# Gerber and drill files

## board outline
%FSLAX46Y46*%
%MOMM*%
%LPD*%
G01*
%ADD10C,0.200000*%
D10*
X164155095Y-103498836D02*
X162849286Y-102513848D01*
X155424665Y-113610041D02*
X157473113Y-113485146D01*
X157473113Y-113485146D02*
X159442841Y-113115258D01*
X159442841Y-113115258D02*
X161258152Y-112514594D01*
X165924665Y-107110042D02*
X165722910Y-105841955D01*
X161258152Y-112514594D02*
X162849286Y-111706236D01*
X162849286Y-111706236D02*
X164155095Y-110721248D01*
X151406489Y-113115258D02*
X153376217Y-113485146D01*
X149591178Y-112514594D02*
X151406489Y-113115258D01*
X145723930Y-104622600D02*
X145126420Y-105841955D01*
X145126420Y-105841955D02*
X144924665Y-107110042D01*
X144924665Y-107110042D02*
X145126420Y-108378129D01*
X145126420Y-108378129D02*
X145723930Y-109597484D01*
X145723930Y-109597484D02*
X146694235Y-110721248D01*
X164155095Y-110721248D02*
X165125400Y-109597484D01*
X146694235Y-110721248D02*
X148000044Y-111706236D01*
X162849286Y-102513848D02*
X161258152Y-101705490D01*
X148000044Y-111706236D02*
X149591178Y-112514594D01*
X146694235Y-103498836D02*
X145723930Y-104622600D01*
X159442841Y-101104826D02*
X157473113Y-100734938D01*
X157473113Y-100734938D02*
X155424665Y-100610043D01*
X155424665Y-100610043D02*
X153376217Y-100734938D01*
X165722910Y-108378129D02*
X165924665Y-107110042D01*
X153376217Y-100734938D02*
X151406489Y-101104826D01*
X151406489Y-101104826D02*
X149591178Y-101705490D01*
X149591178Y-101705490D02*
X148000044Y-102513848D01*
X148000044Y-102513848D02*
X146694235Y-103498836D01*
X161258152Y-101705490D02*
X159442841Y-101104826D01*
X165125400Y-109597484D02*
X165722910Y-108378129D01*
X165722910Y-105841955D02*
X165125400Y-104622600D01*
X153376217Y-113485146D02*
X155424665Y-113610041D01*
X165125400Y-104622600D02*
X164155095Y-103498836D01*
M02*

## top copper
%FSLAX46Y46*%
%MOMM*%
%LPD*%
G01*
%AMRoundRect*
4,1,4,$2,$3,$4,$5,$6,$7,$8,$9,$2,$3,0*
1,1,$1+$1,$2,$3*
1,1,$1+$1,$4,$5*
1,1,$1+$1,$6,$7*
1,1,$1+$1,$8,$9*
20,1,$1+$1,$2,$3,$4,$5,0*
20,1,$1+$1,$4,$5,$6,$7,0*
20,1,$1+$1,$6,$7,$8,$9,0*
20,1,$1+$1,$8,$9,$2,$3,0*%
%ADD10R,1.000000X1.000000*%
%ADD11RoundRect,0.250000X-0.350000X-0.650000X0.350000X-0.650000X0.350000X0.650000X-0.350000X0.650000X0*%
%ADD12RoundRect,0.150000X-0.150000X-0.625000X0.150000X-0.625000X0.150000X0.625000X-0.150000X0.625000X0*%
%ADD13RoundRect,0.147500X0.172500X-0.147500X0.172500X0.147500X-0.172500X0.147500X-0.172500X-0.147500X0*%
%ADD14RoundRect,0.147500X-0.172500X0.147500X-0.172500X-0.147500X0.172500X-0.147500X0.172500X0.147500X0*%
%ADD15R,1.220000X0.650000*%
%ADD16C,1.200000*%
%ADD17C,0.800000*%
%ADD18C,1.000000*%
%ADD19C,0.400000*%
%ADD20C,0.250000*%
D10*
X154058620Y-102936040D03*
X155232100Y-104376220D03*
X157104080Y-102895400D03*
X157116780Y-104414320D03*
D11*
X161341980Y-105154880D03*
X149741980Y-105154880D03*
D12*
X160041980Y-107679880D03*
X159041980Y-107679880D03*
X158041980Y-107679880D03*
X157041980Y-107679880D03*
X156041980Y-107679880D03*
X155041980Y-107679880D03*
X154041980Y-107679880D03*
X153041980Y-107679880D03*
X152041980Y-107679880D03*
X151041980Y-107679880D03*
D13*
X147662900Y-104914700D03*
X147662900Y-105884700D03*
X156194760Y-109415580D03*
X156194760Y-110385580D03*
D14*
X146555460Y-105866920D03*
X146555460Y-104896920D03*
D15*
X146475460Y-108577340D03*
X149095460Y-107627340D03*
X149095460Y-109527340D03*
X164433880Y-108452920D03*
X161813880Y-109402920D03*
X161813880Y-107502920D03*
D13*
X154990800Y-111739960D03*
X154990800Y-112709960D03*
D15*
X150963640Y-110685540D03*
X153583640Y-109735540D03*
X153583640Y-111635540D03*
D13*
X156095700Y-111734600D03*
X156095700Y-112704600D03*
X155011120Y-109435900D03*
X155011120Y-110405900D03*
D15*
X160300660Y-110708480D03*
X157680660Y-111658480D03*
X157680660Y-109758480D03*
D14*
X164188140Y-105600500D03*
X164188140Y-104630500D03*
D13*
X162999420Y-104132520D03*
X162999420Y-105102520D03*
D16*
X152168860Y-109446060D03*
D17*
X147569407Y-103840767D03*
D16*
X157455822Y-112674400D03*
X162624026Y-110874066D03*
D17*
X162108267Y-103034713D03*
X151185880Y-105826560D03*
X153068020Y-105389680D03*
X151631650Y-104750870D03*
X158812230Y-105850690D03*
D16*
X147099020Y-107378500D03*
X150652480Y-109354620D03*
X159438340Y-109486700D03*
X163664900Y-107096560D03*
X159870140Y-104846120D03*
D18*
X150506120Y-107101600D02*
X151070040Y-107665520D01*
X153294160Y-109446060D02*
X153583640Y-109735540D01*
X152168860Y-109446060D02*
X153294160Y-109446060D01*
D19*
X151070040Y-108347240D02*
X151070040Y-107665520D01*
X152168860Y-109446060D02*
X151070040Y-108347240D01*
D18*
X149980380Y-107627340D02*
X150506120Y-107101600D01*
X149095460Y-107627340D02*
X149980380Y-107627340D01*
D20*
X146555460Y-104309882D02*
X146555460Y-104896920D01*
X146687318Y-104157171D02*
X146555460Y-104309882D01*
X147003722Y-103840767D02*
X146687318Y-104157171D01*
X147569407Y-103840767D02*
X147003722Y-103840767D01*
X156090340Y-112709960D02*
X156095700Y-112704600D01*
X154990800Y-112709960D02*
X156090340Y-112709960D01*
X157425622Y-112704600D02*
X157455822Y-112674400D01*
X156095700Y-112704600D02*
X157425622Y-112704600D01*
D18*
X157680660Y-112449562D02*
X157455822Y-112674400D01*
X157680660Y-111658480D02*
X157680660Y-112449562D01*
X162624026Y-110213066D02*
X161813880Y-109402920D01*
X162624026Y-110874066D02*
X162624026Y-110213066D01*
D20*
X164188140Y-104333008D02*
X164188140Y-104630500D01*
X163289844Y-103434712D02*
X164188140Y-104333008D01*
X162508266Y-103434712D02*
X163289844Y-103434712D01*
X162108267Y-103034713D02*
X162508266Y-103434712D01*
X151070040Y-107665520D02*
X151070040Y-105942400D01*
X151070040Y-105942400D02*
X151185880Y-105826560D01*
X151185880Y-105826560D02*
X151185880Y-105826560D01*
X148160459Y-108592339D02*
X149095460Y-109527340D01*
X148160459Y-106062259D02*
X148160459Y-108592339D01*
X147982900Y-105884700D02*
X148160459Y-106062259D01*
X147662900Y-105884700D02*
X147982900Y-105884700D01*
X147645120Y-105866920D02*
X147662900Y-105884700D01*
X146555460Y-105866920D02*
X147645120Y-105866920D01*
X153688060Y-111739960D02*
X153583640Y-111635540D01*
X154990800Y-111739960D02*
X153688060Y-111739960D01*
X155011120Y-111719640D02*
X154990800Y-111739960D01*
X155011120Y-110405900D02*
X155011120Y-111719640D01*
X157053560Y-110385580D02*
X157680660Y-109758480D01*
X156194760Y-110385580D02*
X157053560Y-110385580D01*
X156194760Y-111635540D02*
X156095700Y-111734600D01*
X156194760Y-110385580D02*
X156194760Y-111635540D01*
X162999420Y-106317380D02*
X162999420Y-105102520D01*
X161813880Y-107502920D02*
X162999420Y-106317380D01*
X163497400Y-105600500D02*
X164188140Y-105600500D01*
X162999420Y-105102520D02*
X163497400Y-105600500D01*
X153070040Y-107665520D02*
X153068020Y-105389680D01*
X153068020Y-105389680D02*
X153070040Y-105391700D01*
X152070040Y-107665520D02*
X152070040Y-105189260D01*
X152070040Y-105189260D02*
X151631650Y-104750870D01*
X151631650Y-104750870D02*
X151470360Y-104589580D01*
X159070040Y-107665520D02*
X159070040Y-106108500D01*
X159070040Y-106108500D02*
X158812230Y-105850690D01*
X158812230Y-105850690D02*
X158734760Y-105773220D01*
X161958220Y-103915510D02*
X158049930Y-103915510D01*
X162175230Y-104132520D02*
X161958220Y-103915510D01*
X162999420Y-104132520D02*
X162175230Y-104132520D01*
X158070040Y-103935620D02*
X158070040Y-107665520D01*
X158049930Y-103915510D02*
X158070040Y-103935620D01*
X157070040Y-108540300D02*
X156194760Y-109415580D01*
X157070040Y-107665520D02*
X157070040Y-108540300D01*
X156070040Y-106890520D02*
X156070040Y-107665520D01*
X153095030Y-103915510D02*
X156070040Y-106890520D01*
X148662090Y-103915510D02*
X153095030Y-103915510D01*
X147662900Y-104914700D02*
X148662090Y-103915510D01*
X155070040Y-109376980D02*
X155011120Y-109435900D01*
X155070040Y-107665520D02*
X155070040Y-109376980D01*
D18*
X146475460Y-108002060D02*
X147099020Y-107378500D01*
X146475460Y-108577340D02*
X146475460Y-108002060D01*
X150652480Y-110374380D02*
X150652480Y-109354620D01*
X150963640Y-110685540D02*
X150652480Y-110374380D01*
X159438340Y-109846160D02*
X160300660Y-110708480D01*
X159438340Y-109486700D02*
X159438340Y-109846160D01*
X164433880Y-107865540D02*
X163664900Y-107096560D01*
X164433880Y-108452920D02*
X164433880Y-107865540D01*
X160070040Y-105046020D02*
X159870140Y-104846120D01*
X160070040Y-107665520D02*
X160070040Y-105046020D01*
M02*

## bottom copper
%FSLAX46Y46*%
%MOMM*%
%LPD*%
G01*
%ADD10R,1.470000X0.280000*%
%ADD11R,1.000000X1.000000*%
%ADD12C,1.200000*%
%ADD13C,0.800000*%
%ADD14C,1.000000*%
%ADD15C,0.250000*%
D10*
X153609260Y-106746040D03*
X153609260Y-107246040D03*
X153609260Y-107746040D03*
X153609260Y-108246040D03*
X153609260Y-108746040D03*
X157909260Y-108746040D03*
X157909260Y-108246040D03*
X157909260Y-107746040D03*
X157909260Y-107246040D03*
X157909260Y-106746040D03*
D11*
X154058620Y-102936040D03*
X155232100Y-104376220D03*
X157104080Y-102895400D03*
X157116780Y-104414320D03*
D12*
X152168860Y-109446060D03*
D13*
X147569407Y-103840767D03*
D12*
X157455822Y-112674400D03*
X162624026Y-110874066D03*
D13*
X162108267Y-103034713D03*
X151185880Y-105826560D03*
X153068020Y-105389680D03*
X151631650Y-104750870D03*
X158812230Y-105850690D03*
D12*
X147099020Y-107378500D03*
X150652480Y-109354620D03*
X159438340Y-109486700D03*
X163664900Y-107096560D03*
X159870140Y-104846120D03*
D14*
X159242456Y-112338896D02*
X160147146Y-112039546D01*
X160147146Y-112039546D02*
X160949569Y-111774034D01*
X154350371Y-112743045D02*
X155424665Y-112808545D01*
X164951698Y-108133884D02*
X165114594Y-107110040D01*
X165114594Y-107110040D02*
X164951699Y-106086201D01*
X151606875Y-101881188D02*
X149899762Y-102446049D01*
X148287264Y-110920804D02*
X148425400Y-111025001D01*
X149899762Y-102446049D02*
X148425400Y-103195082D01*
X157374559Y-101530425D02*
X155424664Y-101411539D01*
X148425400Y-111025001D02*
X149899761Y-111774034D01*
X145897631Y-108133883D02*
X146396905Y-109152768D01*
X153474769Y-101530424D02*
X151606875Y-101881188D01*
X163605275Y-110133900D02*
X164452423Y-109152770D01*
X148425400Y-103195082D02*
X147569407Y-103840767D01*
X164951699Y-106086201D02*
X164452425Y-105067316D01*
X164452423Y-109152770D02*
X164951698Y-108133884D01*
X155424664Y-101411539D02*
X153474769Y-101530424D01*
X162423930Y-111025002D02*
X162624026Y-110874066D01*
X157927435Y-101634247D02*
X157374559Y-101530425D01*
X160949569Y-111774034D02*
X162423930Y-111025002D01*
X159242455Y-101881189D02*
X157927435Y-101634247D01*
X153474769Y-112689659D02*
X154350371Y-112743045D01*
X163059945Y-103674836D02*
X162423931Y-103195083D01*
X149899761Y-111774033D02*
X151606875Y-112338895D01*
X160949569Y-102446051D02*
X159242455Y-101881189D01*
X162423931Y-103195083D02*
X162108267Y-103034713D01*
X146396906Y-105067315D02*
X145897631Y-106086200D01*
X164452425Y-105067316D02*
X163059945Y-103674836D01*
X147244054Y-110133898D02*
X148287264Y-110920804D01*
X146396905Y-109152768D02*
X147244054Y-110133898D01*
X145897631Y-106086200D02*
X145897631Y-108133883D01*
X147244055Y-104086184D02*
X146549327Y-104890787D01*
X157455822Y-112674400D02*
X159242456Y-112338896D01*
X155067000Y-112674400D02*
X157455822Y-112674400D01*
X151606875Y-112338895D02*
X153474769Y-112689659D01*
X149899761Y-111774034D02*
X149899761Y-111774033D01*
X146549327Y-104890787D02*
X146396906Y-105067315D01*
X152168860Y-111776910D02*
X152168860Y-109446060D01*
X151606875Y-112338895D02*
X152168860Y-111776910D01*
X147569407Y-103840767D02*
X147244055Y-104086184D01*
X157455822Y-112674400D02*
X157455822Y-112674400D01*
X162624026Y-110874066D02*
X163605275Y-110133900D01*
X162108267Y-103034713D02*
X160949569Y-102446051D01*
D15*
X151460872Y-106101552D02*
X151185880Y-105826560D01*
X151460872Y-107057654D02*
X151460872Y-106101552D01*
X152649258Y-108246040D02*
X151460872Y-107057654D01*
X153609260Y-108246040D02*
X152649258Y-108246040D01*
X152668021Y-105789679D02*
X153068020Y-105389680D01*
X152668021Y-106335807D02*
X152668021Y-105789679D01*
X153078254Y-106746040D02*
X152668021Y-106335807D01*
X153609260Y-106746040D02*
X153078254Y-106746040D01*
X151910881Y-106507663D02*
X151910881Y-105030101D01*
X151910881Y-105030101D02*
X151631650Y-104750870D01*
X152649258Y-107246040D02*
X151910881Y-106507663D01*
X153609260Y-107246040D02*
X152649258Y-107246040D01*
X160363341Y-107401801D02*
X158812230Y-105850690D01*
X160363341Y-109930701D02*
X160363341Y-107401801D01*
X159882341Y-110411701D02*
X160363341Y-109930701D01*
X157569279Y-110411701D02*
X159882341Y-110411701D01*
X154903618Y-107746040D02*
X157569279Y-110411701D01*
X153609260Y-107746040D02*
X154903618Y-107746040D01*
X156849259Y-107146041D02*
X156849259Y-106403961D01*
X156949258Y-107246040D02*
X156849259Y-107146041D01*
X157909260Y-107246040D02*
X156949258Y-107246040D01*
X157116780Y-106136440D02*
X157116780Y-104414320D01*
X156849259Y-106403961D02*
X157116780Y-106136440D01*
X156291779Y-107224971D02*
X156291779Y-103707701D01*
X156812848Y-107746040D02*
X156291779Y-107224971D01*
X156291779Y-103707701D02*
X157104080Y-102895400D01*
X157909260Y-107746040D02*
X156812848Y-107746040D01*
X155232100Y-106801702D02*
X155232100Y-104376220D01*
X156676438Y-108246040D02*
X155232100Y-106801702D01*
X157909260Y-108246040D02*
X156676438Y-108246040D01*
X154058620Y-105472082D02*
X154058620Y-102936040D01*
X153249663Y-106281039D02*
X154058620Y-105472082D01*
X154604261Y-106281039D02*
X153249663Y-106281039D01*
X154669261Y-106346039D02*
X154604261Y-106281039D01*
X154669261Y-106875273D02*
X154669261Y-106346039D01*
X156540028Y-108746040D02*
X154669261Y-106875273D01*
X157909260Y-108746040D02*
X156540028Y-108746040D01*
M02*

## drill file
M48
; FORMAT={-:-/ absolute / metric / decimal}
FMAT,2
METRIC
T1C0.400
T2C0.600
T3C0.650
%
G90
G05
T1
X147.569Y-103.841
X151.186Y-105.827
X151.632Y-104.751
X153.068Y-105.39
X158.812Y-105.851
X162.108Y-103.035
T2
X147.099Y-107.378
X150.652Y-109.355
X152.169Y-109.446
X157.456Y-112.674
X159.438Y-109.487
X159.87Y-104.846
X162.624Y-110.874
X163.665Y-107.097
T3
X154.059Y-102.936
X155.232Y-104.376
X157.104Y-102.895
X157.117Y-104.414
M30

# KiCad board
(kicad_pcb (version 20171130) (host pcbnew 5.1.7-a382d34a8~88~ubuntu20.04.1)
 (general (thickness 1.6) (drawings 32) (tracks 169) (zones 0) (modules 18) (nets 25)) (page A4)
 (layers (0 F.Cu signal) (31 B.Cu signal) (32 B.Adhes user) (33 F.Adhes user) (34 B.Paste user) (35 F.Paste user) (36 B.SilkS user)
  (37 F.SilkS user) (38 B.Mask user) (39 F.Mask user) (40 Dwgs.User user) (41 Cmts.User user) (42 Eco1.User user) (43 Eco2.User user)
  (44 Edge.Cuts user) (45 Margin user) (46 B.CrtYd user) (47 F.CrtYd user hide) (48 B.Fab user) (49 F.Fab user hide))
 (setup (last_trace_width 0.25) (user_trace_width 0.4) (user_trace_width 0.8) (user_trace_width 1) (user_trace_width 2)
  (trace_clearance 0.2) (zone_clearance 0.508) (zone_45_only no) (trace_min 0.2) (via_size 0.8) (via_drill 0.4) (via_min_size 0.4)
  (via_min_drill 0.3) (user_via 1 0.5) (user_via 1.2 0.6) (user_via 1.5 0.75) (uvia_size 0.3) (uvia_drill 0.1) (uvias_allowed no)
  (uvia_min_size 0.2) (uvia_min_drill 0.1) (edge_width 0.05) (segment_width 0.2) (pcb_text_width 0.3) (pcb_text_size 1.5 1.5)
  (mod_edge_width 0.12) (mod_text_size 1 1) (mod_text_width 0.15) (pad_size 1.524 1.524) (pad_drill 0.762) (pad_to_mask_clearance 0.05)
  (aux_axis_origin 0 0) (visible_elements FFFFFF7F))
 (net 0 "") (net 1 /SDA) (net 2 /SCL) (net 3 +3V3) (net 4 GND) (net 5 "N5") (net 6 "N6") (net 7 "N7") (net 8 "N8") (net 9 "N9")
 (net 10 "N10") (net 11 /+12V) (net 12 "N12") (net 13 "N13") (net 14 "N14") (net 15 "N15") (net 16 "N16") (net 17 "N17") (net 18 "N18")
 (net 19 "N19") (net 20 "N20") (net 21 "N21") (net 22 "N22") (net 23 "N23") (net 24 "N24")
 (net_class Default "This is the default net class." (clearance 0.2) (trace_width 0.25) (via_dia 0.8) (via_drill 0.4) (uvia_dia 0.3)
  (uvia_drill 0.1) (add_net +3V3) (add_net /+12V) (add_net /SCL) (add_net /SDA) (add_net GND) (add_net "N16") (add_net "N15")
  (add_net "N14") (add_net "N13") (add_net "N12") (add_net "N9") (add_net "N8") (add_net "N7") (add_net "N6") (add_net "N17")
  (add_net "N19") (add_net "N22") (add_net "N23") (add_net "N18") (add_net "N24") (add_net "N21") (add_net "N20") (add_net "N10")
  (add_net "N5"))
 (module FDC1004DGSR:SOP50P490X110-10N (layer B.Cu) (at 155.75926 107.74604 180)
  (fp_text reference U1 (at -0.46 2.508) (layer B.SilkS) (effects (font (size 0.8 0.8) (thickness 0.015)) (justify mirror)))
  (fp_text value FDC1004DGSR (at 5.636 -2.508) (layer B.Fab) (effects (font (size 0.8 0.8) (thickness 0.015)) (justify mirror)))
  (pad 10 smd rect (at 2.15 1 180) (size 1.47 0.28) (layers B.Cu B.Paste B.Mask) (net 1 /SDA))
  (pad 9 smd rect (at 2.15 0.5 180) (size 1.47 0.28) (layers B.Cu B.Paste B.Mask) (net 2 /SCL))
  (pad 8 smd rect (at 2.15 0 180) (size 1.47 0.28) (layers B.Cu B.Paste B.Mask) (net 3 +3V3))
  (pad 7 smd rect (at 2.15 -0.5 180) (size 1.47 0.28) (layers B.Cu B.Paste B.Mask) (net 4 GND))
  (pad 6 smd rect (at 2.15 -1 180) (size 1.47 0.28) (layers B.Cu B.Paste B.Mask) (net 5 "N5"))
  (pad 5 smd rect (at -2.15 -1 180) (size 1.47 0.28) (layers B.Cu B.Paste B.Mask) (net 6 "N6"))
  (pad 4 smd rect (at -2.15 -0.5 180) (size 1.47 0.28) (layers B.Cu B.Paste B.Mask) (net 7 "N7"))
  (pad 3 smd rect (at -2.15 0 180) (size 1.47 0.28) (layers B.Cu B.Paste B.Mask) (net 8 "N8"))
  (pad 2 smd rect (at -2.15 0.5 180) (size 1.47 0.28) (layers B.Cu B.Paste B.Mask) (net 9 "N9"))
  (pad 1 smd rect (at -2.15 1 180) (size 1.47 0.28) (layers B.Cu B.Paste B.Mask) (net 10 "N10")))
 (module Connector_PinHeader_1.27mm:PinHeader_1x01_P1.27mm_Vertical (layer F.Cu) (at 154.05862 102.93604)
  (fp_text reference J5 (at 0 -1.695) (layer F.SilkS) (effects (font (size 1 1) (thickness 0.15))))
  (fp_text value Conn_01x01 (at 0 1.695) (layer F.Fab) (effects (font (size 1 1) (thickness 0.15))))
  (pad 1 thru_hole rect (at 0 0) (size 1 1) (drill 0.65) (layers *.Cu *.Mask) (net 6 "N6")))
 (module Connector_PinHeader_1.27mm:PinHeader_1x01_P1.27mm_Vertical (layer F.Cu) (at 155.2321 104.37622)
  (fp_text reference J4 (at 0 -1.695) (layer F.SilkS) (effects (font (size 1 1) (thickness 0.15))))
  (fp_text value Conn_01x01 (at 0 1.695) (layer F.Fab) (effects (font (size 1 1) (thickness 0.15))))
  (pad 1 thru_hole rect (at 0 0) (size 1 1) (drill 0.65) (layers *.Cu *.Mask) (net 7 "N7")))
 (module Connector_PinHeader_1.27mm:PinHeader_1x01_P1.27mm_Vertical (layer F.Cu) (at 157.10408 102.8954)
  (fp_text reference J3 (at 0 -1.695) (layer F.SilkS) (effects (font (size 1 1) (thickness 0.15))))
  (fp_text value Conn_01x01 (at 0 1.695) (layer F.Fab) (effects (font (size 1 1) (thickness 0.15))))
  (pad 1 thru_hole rect (at 0 0) (size 1 1) (drill 0.65) (layers *.Cu *.Mask) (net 8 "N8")))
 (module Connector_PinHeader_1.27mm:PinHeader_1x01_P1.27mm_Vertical (layer F.Cu) (at 157.11678 104.41432)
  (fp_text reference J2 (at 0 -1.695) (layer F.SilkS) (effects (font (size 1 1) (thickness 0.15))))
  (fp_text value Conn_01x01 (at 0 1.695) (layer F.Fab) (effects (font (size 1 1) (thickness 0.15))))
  (pad 1 thru_hole rect (at 0 0) (size 1 1) (drill 0.65) (layers *.Cu *.Mask) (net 9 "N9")))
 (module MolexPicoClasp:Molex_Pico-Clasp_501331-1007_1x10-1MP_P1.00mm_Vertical (layer F.Cu) (at 155.54198 106.35488)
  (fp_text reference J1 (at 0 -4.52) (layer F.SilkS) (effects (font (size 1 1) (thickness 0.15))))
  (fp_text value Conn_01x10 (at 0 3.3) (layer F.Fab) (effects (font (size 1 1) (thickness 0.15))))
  (pad MP smd roundrect (at 5.8 -1.2) (size 1.2 1.8) (layers F.Cu F.Paste F.Mask) (roundrect_rratio 0.208333))
  (pad MP smd roundrect (at -5.8 -1.2) (size 1.2 1.8) (layers F.Cu F.Paste F.Mask) (roundrect_rratio 0.208333))
  (pad 10 smd roundrect (at 4.5 1.325) (size 0.6 1.55) (layers F.Cu F.Paste F.Mask) (roundrect_rratio 0.25) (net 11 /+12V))
  (pad 9 smd roundrect (at 3.5 1.325) (size 0.6 1.55) (layers F.Cu F.Paste F.Mask) (roundrect_rratio 0.25) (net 3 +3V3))
  (pad 8 smd roundrect (at 2.5 1.325) (size 0.6 1.55) (layers F.Cu F.Paste F.Mask) (roundrect_rratio 0.25) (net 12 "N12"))
  (pad 7 smd roundrect (at 1.5 1.325) (size 0.6 1.55) (layers F.Cu F.Paste F.Mask) (roundrect_rratio 0.25) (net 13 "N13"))
  (pad 6 smd roundrect (at 0.5 1.325) (size 0.6 1.55) (layers F.Cu F.Paste F.Mask) (roundrect_rratio 0.25) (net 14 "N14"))
  (pad 5 smd roundrect (at -0.5 1.325) (size 0.6 1.55) (layers F.Cu F.Paste F.Mask) (roundrect_rratio 0.25) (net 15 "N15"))
  (pad 4 smd roundrect (at -1.5 1.325) (size 0.6 1.55) (layers F.Cu F.Paste F.Mask) (roundrect_rratio 0.25) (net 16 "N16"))
  (pad 3 smd roundrect (at -2.5 1.325) (size 0.6 1.55) (layers F.Cu F.Paste F.Mask) (roundrect_rratio 0.25) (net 1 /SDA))
  (pad 2 smd roundrect (at -3.5 1.325) (size 0.6 1.55) (layers F.Cu F.Paste F.Mask) (roundrect_rratio 0.25) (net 2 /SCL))
  (pad 1 smd roundrect (at -4.5 1.325) (size 0.6 1.55) (layers F.Cu F.Paste F.Mask) (roundrect_rratio 0.25) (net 4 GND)))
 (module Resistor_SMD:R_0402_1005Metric (layer F.Cu) (at 147.6629 105.3997 90)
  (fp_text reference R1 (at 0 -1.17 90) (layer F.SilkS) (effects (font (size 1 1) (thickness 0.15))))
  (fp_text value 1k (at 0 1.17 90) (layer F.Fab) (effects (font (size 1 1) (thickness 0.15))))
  (pad 2 smd roundrect (at 0.485 0 90) (size 0.59 0.64) (layers F.Cu F.Paste F.Mask) (roundrect_rratio 0.25) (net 14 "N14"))
  (pad 1 smd roundrect (at -0.485 0 90) (size 0.59 0.64) (layers F.Cu F.Paste F.Mask) (roundrect_rratio 0.25) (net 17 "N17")))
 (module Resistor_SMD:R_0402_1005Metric (layer F.Cu) (at 156.19476 109.90058 90)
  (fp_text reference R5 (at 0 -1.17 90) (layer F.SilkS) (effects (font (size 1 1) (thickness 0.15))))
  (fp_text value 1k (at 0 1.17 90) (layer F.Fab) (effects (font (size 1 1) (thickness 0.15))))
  (pad 2 smd roundrect (at 0.485 0 90) (size 0.59 0.64) (layers F.Cu F.Paste F.Mask) (roundrect_rratio 0.25) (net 13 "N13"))
  (pad 1 smd roundrect (at -0.485 0 90) (size 0.59 0.64) (layers F.Cu F.Paste F.Mask) (roundrect_rratio 0.25) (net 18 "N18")))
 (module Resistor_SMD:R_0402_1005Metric (layer F.Cu) (at 146.55546 105.38192 270)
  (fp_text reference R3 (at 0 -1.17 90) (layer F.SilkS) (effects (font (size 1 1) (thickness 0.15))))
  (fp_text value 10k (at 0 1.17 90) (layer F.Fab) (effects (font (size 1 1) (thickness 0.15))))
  (pad 2 smd roundrect (at 0.485 0 270) (size 0.59 0.64) (layers F.Cu F.Paste F.Mask) (roundrect_rratio 0.25) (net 17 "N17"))
  (pad 1 smd roundrect (at -0.485 0 270) (size 0.59 0.64) (layers F.Cu F.Paste F.Mask) (roundrect_rratio 0.25) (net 4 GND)))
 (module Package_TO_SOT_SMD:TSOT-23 (layer F.Cu) (at 147.78546 108.57734 180)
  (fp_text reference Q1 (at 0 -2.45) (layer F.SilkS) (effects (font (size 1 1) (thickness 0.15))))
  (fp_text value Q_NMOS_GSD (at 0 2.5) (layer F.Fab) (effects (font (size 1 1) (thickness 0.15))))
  (pad 3 smd rect (at 1.31 0 180) (size 1.22 0.65) (layers F.Cu F.Paste F.Mask) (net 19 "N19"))
  (pad 2 smd rect (at -1.31 0.95 180) (size 1.22 0.65) (layers F.Cu F.Paste F.Mask) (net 4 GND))
  (pad 1 smd rect (at -1.31 -0.95 180) (size 1.22 0.65) (layers F.Cu F.Paste F.Mask) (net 17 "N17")))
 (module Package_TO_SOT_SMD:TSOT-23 (layer F.Cu) (at 163.12388 108.45292)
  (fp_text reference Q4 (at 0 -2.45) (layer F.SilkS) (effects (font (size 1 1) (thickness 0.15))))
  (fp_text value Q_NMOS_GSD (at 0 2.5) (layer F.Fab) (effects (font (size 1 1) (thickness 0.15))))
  (pad 3 smd rect (at 1.31 0) (size 1.22 0.65) (layers F.Cu F.Paste F.Mask) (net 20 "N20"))
  (pad 2 smd rect (at -1.31 0.95) (size 1.22 0.65) (layers F.Cu F.Paste F.Mask) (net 4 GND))
  (pad 1 smd rect (at -1.31 -0.95) (size 1.22 0.65) (layers F.Cu F.Paste F.Mask) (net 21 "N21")))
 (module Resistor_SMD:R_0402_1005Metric (layer F.Cu) (at 154.9908 112.22496 90)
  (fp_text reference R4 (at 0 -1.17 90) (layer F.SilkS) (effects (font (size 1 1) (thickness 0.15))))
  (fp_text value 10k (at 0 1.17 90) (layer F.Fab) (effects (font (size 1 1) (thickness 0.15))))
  (pad 2 smd roundrect (at 0.485 0 90) (size 0.59 0.64) (layers F.Cu F.Paste F.Mask) (roundrect_rratio 0.25) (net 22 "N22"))
  (pad 1 smd roundrect (at -0.485 0 90) (size 0.59 0.64) (layers F.Cu F.Paste F.Mask) (roundrect_rratio 0.25) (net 4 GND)))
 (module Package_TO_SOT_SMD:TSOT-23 (layer F.Cu) (at 152.27364 110.68554 180)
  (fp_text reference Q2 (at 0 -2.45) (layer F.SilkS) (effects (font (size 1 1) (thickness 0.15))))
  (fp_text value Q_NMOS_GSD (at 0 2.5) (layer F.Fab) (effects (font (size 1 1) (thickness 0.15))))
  (pad 3 smd rect (at 1.31 0 180) (size 1.22 0.65) (layers F.Cu F.Paste F.Mask) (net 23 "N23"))
  (pad 2 smd rect (at -1.31 0.95 180) (size 1.22 0.65) (layers F.Cu F.Paste F.Mask) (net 4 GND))
  (pad 1 smd rect (at -1.31 -0.95 180) (size 1.22 0.65) (layers F.Cu F.Paste F.Mask) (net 22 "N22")))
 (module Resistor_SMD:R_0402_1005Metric (layer F.Cu) (at 156.0957 112.2196 90)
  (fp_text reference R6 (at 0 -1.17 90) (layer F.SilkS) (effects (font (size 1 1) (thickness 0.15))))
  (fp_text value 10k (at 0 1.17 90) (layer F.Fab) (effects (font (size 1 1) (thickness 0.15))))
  (pad 2 smd roundrect (at 0.485 0 90) (size 0.59 0.64) (layers F.Cu F.Paste F.Mask) (roundrect_rratio 0.25) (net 18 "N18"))
  (pad 1 smd roundrect (at -0.485 0 90) (size 0.59 0.64) (layers F.Cu F.Paste F.Mask) (roundrect_rratio 0.25) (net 4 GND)))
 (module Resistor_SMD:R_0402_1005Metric (layer F.Cu) (at 155.01112 109.9209 90)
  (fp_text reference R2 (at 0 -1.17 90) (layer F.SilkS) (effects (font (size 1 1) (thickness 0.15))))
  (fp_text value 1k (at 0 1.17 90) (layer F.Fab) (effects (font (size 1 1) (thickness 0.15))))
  (pad 2 smd roundrect (at 0.485 0 90) (size 0.59 0.64) (layers F.Cu F.Paste F.Mask) (roundrect_rratio 0.25) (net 15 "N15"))
  (pad 1 smd roundrect (at -0.485 0 90) (size 0.59 0.64) (layers F.Cu F.Paste F.Mask) (roundrect_rratio 0.25) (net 22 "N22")))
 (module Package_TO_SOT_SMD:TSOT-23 (layer F.Cu) (at 158.99066 110.70848)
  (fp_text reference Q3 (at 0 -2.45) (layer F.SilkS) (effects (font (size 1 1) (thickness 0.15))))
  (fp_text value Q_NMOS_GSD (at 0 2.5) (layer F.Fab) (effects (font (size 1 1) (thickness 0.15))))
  (pad 3 smd rect (at 1.31 0) (size 1.22 0.65) (layers F.Cu F.Paste F.Mask) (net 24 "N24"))
  (pad 2 smd rect (at -1.31 0.95) (size 1.22 0.65) (layers F.Cu F.Paste F.Mask) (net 4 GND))
  (pad 1 smd rect (at -1.31 -0.95) (size 1.22 0.65) (layers F.Cu F.Paste F.Mask) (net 18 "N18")))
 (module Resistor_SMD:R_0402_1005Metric (layer F.Cu) (at 164.18814 105.1155 270)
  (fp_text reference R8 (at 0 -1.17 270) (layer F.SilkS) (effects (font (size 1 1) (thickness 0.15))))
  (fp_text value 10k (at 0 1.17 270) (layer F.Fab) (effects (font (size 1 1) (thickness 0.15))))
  (pad 2 smd roundrect (at 0.485 0 270) (size 0.59 0.64) (layers F.Cu F.Paste F.Mask) (roundrect_rratio 0.25) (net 21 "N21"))
  (pad 1 smd roundrect (at -0.485 0 270) (size 0.59 0.64) (layers F.Cu F.Paste F.Mask) (roundrect_rratio 0.25) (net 4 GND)))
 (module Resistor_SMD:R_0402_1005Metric (layer F.Cu) (at 162.99942 104.61752 90)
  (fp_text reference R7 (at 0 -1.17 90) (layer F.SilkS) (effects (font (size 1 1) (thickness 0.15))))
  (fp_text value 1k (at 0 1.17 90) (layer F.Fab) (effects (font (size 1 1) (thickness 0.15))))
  (pad 2 smd roundrect (at 0.485 0 90) (size 0.59 0.64) (layers F.Cu F.Paste F.Mask) (roundrect_rratio 0.25) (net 12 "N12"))
  (pad 1 smd roundrect (at -0.485 0 90) (size 0.59 0.64) (layers F.Cu F.Paste F.Mask) (roundrect_rratio 0.25) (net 21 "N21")))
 (gr_line (start 164.155095 103.498836) (end 162.849286 102.513848) (layer Edge.Cuts) (width 0.2))
 (gr_line (start 155.424665 113.610041) (end 157.473113 113.485146) (layer Edge.Cuts) (width 0.2))
 (gr_line (start 157.473113 113.485146) (end 159.442841 113.115258) (layer Edge.Cuts) (width 0.2))
 (gr_line (start 159.442841 113.115258) (end 161.258152 112.514594) (layer Edge.Cuts) (width 0.2))
 (gr_line (start 165.924665 107.110042) (end 165.72291 105.841955) (layer Edge.Cuts) (width 0.2))
 (gr_line (start 161.258152 112.514594) (end 162.849286 111.706236) (layer Edge.Cuts) (width 0.2))
 (gr_line (start 162.849286 111.706236) (end 164.155095 110.721248) (layer Edge.Cuts) (width 0.2))
 (gr_line (start 151.406489 113.115258) (end 153.376217 113.485146) (layer Edge.Cuts) (width 0.2))
 (gr_line (start 149.591178 112.514594) (end 151.406489 113.115258) (layer Edge.Cuts) (width 0.2))
 (gr_line (start 145.72393 104.6226) (end 145.12642 105.841955) (layer Edge.Cuts) (width 0.2))
 (gr_line (start 145.12642 105.841955) (end 144.924665 107.110042) (layer Edge.Cuts) (width 0.2))
 (gr_line (start 144.924665 107.110042) (end 145.12642 108.378129) (layer Edge.Cuts) (width 0.2))
 (gr_line (start 145.12642 108.378129) (end 145.72393 109.597484) (layer Edge.Cuts) (width 0.2))
 (gr_line (start 145.72393 109.597484) (end 146.694235 110.721248) (layer Edge.Cuts) (width 0.2))
 (gr_line (start 164.155095 110.721248) (end 165.1254 109.597484) (layer Edge.Cuts) (width 0.2))
 (gr_line (start 146.694235 110.721248) (end 148.000044 111.706236) (layer Edge.Cuts) (width 0.2))
 (gr_line (start 162.849286 102.513848) (end 161.258152 101.70549) (layer Edge.Cuts) (width 0.2))
 (gr_line (start 148.000044 111.706236) (end 149.591178 112.514594) (layer Edge.Cuts) (width 0.2))
 (gr_line (start 146.694235 103.498836) (end 145.72393 104.6226) (layer Edge.Cuts) (width 0.2))
 (gr_line (start 159.442841 101.104826) (end 157.473113 100.734938) (layer Edge.Cuts) (width 0.2))
 (gr_line (start 157.473113 100.734938) (end 155.424665 100.610043) (layer Edge.Cuts) (width 0.2))
 (gr_line (start 155.424665 100.610043) (end 153.376217 100.734938) (layer Edge.Cuts) (width 0.2))
 (gr_line (start 165.72291 108.378129) (end 165.924665 107.110042) (layer Edge.Cuts) (width 0.2))
 (gr_line (start 153.376217 100.734938) (end 151.406489 101.104826) (layer Edge.Cuts) (width 0.2))
 (gr_line (start 151.406489 101.104826) (end 149.591178 101.70549) (layer Edge.Cuts) (width 0.2))
 (gr_line (start 149.591178 101.70549) (end 148.000044 102.513848) (layer Edge.Cuts) (width 0.2))
 (gr_line (start 148.000044 102.513848) (end 146.694235 103.498836) (layer Edge.Cuts) (width 0.2))
 (gr_line (start 161.258152 101.70549) (end 159.442841 101.104826) (layer Edge.Cuts) (width 0.2))
 (gr_line (start 165.1254 109.597484) (end 165.72291 108.378129) (layer Edge.Cuts) (width 0.2))
 (gr_line (start 165.72291 105.841955) (end 165.1254 104.6226) (layer Edge.Cuts) (width 0.2))
 (gr_line (start 153.376217 113.485146) (end 155.424665 113.610041) (layer Edge.Cuts) (width 0.2))
 (gr_line (start 165.1254 104.6226) (end 164.155095 103.498836) (layer Edge.Cuts) (width 0.2))
 (via (at 152.16886 109.44606) (size 1.2) (drill 0.6) (layers F.Cu B.Cu) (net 4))
 (segment (start 159.242456 112.338896) (end 160.147146 112.039546) (width 1) (layer B.Cu) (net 4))
 (segment (start 160.147146 112.039546) (end 160.949569 111.774034) (width 1) (layer B.Cu) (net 4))
 (segment (start 154.350371 112.743045) (end 155.424665 112.808545) (width 1) (layer B.Cu) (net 4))
 (segment (start 164.951698 108.133884) (end 165.114594 107.11004) (width 1) (layer B.Cu) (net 4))
 (segment (start 165.114594 107.11004) (end 164.951699 106.086201) (width 1) (layer B.Cu) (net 4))
 (segment (start 151.606875 101.881188) (end 149.899762 102.446049) (width 1) (layer B.Cu) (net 4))
 (segment (start 148.287264 110.920804) (end 148.4254 111.025001) (width 1) (layer B.Cu) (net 4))
 (segment (start 149.899762 102.446049) (end 148.4254 103.195082) (width 1) (layer B.Cu) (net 4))
 (segment (start 157.374559 101.530425) (end 155.424664 101.411539) (width 1) (layer B.Cu) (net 4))
 (segment (start 148.4254 111.025001) (end 149.899761 111.774034) (width 1) (layer B.Cu) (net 4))
 (segment (start 145.897631 108.133883) (end 146.396905 109.152768) (width 1) (layer B.Cu) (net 4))
 (segment (start 153.474769 101.530424) (end 151.606875 101.881188) (width 1) (layer B.Cu) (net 4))
 (segment (start 163.605275 110.1339) (end 164.452423 109.15277) (width 1) (layer B.Cu) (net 4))
 (segment (start 148.4254 103.195082) (end 147.569407 103.840767) (width 1) (layer B.Cu) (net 4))
 (segment (start 164.951699 106.086201) (end 164.452425 105.067316) (width 1) (layer B.Cu) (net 4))
 (segment (start 164.452423 109.15277) (end 164.951698 108.133884) (width 1) (layer B.Cu) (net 4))
 (segment (start 155.424664 101.411539) (end 153.474769 101.530424) (width 1) (layer B.Cu) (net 4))
 (segment (start 162.42393 111.025002) (end 162.624026 110.874066) (width 1) (layer B.Cu) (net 4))
 (segment (start 157.927435 101.634247) (end 157.374559 101.530425) (width 1) (layer B.Cu) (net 4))
 (segment (start 160.949569 111.774034) (end 162.42393 111.025002) (width 1) (layer B.Cu) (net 4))
 (segment (start 159.242455 101.881189) (end 157.927435 101.634247) (width 1) (layer B.Cu) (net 4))
 (segment (start 153.474769 112.689659) (end 154.350371 112.743045) (width 1) (layer B.Cu) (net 4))
 (segment (start 163.059945 103.674836) (end 162.423931 103.195083) (width 1) (layer B.Cu) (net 4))
 (segment (start 149.899761 111.774033) (end 151.606875 112.338895) (width 1) (layer B.Cu) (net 4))
 (segment (start 160.949569 102.446051) (end 159.242455 101.881189) (width 1) (layer B.Cu) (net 4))
 (segment (start 162.423931 103.195083) (end 162.108267 103.034713) (width 1) (layer B.Cu) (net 4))
 (segment (start 146.396906 105.067315) (end 145.897631 106.0862) (width 1) (layer B.Cu) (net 4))
 (segment (start 164.452425 105.067316) (end 163.059945 103.674836) (width 1) (layer B.Cu) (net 4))
 (segment (start 147.244054 110.133898) (end 148.287264 110.920804) (width 1) (layer B.Cu) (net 4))
 (segment (start 146.396905 109.152768) (end 147.244054 110.133898) (width 1) (layer B.Cu) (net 4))
 (segment (start 145.897631 106.0862) (end 145.897631 108.133883) (width 1) (layer B.Cu) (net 4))
 (segment (start 147.244055 104.086184) (end 146.549327 104.890787) (width 1) (layer B.Cu) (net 4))
 (segment (start 157.455822 112.6744) (end 159.242456 112.338896) (width 1) (layer B.Cu) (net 4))
 (segment (start 155.067 112.6744) (end 157.455822 112.6744) (width 1) (layer B.Cu) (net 4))
 (segment (start 151.606875 112.338895) (end 153.474769 112.689659) (width 1) (layer B.Cu) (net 4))
 (segment (start 149.899761 111.774034) (end 149.899761 111.774033) (width 1) (layer B.Cu) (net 4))
 (segment (start 146.549327 104.890787) (end 146.396906 105.067315) (width 1) (layer B.Cu) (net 4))
 (segment (start 150.50612 107.1016) (end 151.07004 107.66552) (width 1) (layer F.Cu) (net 4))
 (segment (start 153.29416 109.44606) (end 153.58364 109.73554) (width 1) (layer F.Cu) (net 4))
 (segment (start 152.16886 109.44606) (end 153.29416 109.44606) (width 1) (layer F.Cu) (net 4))
 (segment (start 151.07004 108.34724) (end 151.07004 107.66552) (width 0.4) (layer F.Cu) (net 4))
 (segment (start 152.16886 109.44606) (end 151.07004 108.34724) (width 0.4) (layer F.Cu) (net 4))
 (segment (start 152.16886 111.77691) (end 152.16886 109.44606) (width 1) (layer B.Cu) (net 4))
 (segment (start 151.606875 112.338895) (end 152.16886 111.77691) (width 1) (layer B.Cu) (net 4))
 (segment (start 149.98038 107.62734) (end 150.50612 107.1016) (width 1) (layer F.Cu) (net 4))
 (segment (start 149.09546 107.62734) (end 149.98038 107.62734) (width 1) (layer F.Cu) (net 4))
 (segment (start 147.569407 103.840767) (end 147.244055 104.086184) (width 1) (layer B.Cu) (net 4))
 (via (at 147.569407 103.840767) (size 0.8) (drill 0.4) (layers F.Cu B.Cu) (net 4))
 (segment (start 146.55546 104.309882) (end 146.55546 104.89692) (width 0.25) (layer F.Cu) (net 4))
 (segment (start 146.687318 104.157171) (end 146.55546 104.309882) (width 0.25) (layer F.Cu) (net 4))
 (segment (start 147.003722 103.840767) (end 146.687318 104.157171) (width 0.25) (layer F.Cu) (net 4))
 (segment (start 147.569407 103.840767) (end 147.003722 103.840767) (width 0.25) (layer F.Cu) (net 4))
 (segment (start 157.455822 112.6744) (end 157.455822 112.6744) (width 1) (layer B.Cu) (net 4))
 (via (at 157.455822 112.6744) (size 1.2) (drill 0.6) (layers F.Cu B.Cu) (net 4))
 (segment (start 156.09034 112.70996) (end 156.0957 112.7046) (width 0.25) (layer F.Cu) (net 4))
 (segment (start 154.9908 112.70996) (end 156.09034 112.70996) (width 0.25) (layer F.Cu) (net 4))
 (segment (start 157.425622 112.7046) (end 157.455822 112.6744) (width 0.25) (layer F.Cu) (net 4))
 (segment (start 156.0957 112.7046) (end 157.425622 112.7046) (width 0.25) (layer F.Cu) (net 4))
 (segment (start 157.68066 112.449562) (end 157.455822 112.6744) (width 1) (layer F.Cu) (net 4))
 (segment (start 157.68066 111.65848) (end 157.68066 112.449562) (width 1) (layer F.Cu) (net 4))
 (segment (start 162.624026 110.874066) (end 163.605275 110.1339) (width 1) (layer B.Cu) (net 4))
 (via (at 162.624026 110.874066) (size 1.2) (drill 0.6) (layers F.Cu B.Cu) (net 4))
 (segment (start 162.624026 110.213066) (end 161.81388 109.40292) (width 1) (layer F.Cu) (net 4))
 (segment (start 162.624026 110.874066) (end 162.624026 110.213066) (width 1) (layer F.Cu) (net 4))
 (segment (start 162.108267 103.034713) (end 160.949569 102.446051) (width 1) (layer B.Cu) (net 4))
 (via (at 162.108267 103.034713) (size 0.8) (drill 0.4) (layers F.Cu B.Cu) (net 4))
 (segment (start 164.18814 104.333008) (end 164.18814 104.6305) (width 0.25) (layer F.Cu) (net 4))
 (segment (start 163.289844 103.434712) (end 164.18814 104.333008) (width 0.25) (layer F.Cu) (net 4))
 (segment (start 162.508266 103.434712) (end 163.289844 103.434712) (width 0.25) (layer F.Cu) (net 4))
 (segment (start 162.108267 103.034713) (end 162.508266 103.434712) (width 0.25) (layer F.Cu) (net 4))
 (segment (start 151.07004 107.66552) (end 151.07004 105.9424) (width 0.25) (layer F.Cu) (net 4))
 (segment (start 151.07004 105.9424) (end 151.18588 105.82656) (width 0.25) (layer F.Cu) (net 4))
 (segment (start 151.18588 105.82656) (end 151.18588 105.82656) (width 0.25) (layer F.Cu) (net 4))
 (via (at 151.18588 105.82656) (size 0.8) (drill 0.4) (layers F.Cu B.Cu) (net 4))
 (segment (start 151.460872 106.101552) (end 151.18588 105.82656) (width 0.25) (layer B.Cu) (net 4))
 (segment (start 151.460872 107.057654) (end 151.460872 106.101552) (width 0.25) (layer B.Cu) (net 4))
 (segment (start 152.649258 108.24604) (end 151.460872 107.057654) (width 0.25) (layer B.Cu) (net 4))
 (segment (start 153.60926 108.24604) (end 152.649258 108.24604) (width 0.25) (layer B.Cu) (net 4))
 (segment (start 148.160459 108.592339) (end 149.09546 109.52734) (width 0.25) (layer F.Cu) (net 17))
 (segment (start 148.160459 106.062259) (end 148.160459 108.592339) (width 0.25) (layer F.Cu) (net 17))
 (segment (start 147.9829 105.8847) (end 148.160459 106.062259) (width 0.25) (layer F.Cu) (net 17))
 (segment (start 147.6629 105.8847) (end 147.9829 105.8847) (width 0.25) (layer F.Cu) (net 17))
 (segment (start 147.64512 105.86692) (end 147.6629 105.8847) (width 0.25) (layer F.Cu) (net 17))
 (segment (start 146.55546 105.86692) (end 147.64512 105.86692) (width 0.25) (layer F.Cu) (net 17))
 (segment (start 153.68806 111.73996) (end 153.58364 111.63554) (width 0.25) (layer F.Cu) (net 22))
 (segment (start 154.9908 111.73996) (end 153.68806 111.73996) (width 0.25) (layer F.Cu) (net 22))
 (segment (start 155.01112 111.71964) (end 154.9908 111.73996) (width 0.25) (layer F.Cu) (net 22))
 (segment (start 155.01112 110.4059) (end 155.01112 111.71964) (width 0.25) (layer F.Cu) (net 22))
 (segment (start 157.05356 110.38558) (end 157.68066 109.75848) (width 0.25) (layer F.Cu) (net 18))
 (segment (start 156.19476 110.38558) (end 157.05356 110.38558) (width 0.25) (layer F.Cu) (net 18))
 (segment (start 156.19476 111.63554) (end 156.0957 111.7346) (width 0.25) (layer F.Cu) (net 18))
 (segment (start 156.19476 110.38558) (end 156.19476 111.63554) (width 0.25) (layer F.Cu) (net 18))
 (segment (start 162.99942 106.31738) (end 162.99942 105.10252) (width 0.25) (layer F.Cu) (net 21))
 (segment (start 161.81388 107.50292) (end 162.99942 106.31738) (width 0.25) (layer F.Cu) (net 21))
 (segment (start 163.4974 105.6005) (end 164.18814 105.6005) (width 0.25) (layer F.Cu) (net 21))
 (segment (start 162.99942 105.10252) (end 163.4974 105.6005) (width 0.25) (layer F.Cu) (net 21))
 (segment (start 153.07004 107.66552) (end 153.06802 105.38968) (width 0.25) (layer F.Cu) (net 1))
 (segment (start 153.06802 105.38968) (end 153.07004 105.3917) (width 0.25) (layer F.Cu) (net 1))
 (via (at 153.06802 105.38968) (size 0.8) (drill 0.4) (layers F.Cu B.Cu) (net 1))
 (segment (start 152.668021 105.789679) (end 153.06802 105.38968) (width 0.25) (layer B.Cu) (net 1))
 (segment (start 152.668021 106.335807) (end 152.668021 105.789679) (width 0.25) (layer B.Cu) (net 1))
 (segment (start 153.078254 106.74604) (end 152.668021 106.335807) (width 0.25) (layer B.Cu) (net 1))
 (segment (start 153.60926 106.74604) (end 153.078254 106.74604) (width 0.25) (layer B.Cu) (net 1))
 (segment (start 152.07004 107.66552) (end 152.07004 105.18926) (width 0.25) (layer F.Cu) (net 2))
 (segment (start 152.07004 105.18926) (end 151.63165 104.75087) (width 0.25) (layer F.Cu) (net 2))
 (segment (start 151.63165 104.75087) (end 151.47036 104.58958) (width 0.25) (layer F.Cu) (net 2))
 (via (at 151.63165 104.75087) (size 0.8) (drill 0.4) (layers F.Cu B.Cu) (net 2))
 (segment (start 151.910881 106.507663) (end 151.910881 105.030101) (width 0.25) (layer B.Cu) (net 2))
 (segment (start 151.910881 105.030101) (end 151.63165 104.75087) (width 0.25) (layer B.Cu) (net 2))
 (segment (start 152.649258 107.24604) (end 151.910881 106.507663) (width 0.25) (layer B.Cu) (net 2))
 (segment (start 153.60926 107.24604) (end 152.649258 107.24604) (width 0.25) (layer B.Cu) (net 2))
 (segment (start 159.07004 107.66552) (end 159.07004 106.1085) (width 0.25) (layer F.Cu) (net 3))
 (segment (start 159.07004 106.1085) (end 158.81223 105.85069) (width 0.25) (layer F.Cu) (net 3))
 (segment (start 158.81223 105.85069) (end 158.73476 105.77322) (width 0.25) (layer F.Cu) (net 3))
 (via (at 158.81223 105.85069) (size 0.8) (drill 0.4) (layers F.Cu B.Cu) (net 3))
 (segment (start 160.363341 107.401801) (end 158.81223 105.85069) (width 0.25) (layer B.Cu) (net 3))
 (segment (start 160.363341 109.930701) (end 160.363341 107.401801) (width 0.25) (layer B.Cu) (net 3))
 (segment (start 159.882341 110.411701) (end 160.363341 109.930701) (width 0.25) (layer B.Cu) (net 3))
 (segment (start 157.569279 110.411701) (end 159.882341 110.411701) (width 0.25) (layer B.Cu) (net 3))
 (segment (start 154.903618 107.74604) (end 157.569279 110.411701) (width 0.25) (layer B.Cu) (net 3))
 (segment (start 153.60926 107.74604) (end 154.903618 107.74604) (width 0.25) (layer B.Cu) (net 3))
 (segment (start 161.95822 103.91551) (end 158.04993 103.91551) (width 0.25) (layer F.Cu) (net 12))
 (segment (start 162.17523 104.13252) (end 161.95822 103.91551) (width 0.25) (layer F.Cu) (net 12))
 (segment (start 162.99942 104.13252) (end 162.17523 104.13252) (width 0.25) (layer F.Cu) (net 12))
 (segment (start 158.07004 103.93562) (end 158.07004 107.66552) (width 0.25) (layer F.Cu) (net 12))
 (segment (start 158.04993 103.91551) (end 158.07004 103.93562) (width 0.25) (layer F.Cu) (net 12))
 (segment (start 157.07004 108.5403) (end 156.19476 109.41558) (width 0.25) (layer F.Cu) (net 13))
 (segment (start 157.07004 107.66552) (end 157.07004 108.5403) (width 0.25) (layer F.Cu) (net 13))
 (segment (start 156.07004 106.89052) (end 156.07004 107.66552) (width 0.25) (layer F.Cu) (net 14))
 (segment (start 153.09503 103.91551) (end 156.07004 106.89052) (width 0.25) (layer F.Cu) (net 14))
 (segment (start 148.66209 103.91551) (end 153.09503 103.91551) (width 0.25) (layer F.Cu) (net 14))
 (segment (start 147.6629 104.9147) (end 148.66209 103.91551) (width 0.25) (layer F.Cu) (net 14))
 (segment (start 155.07004 109.37698) (end 155.01112 109.4359) (width 0.25) (layer F.Cu) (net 15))
 (segment (start 155.07004 107.66552) (end 155.07004 109.37698) (width 0.25) (layer F.Cu) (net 15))
 (via (at 147.09902 107.3785) (size 1.2) (drill 0.6) (layers F.Cu B.Cu) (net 19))
 (segment (start 146.47546 108.00206) (end 147.09902 107.3785) (width 1) (layer F.Cu) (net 19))
 (segment (start 146.47546 108.57734) (end 146.47546 108.00206) (width 1) (layer F.Cu) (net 19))
 (via (at 150.65248 109.35462) (size 1.2) (drill 0.6) (layers F.Cu B.Cu) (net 23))
 (segment (start 150.65248 110.37438) (end 150.65248 109.35462) (width 1) (layer F.Cu) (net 23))
 (segment (start 150.96364 110.68554) (end 150.65248 110.37438) (width 1) (layer F.Cu) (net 23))
 (via (at 159.43834 109.4867) (size 1.2) (drill 0.6) (layers F.Cu B.Cu) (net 24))
 (segment (start 159.43834 109.84616) (end 160.30066 110.70848) (width 1) (layer F.Cu) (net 24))
 (segment (start 159.43834 109.4867) (end 159.43834 109.84616) (width 1) (layer F.Cu) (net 24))
 (via (at 163.6649 107.09656) (size 1.2) (drill 0.6) (layers F.Cu B.Cu) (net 20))
 (segment (start 164.43388 107.86554) (end 163.6649 107.09656) (width 1) (layer F.Cu) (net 20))
 (segment (start 164.43388 108.45292) (end 164.43388 107.86554) (width 1) (layer F.Cu) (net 20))
 (via (at 159.87014 104.84612) (size 1.2) (drill 0.6) (layers F.Cu B.Cu) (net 11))
 (segment (start 160.07004 105.04602) (end 159.87014 104.84612) (width 1) (layer F.Cu) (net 11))
 (segment (start 160.07004 107.66552) (end 160.07004 105.04602) (width 1) (layer F.Cu) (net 11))
 (segment (start 156.849259 107.146041) (end 156.849259 106.403961) (width 0.25) (layer B.Cu) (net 9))
 (segment (start 156.949258 107.24604) (end 156.849259 107.146041) (width 0.25) (layer B.Cu) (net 9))
 (segment (start 157.90926 107.24604) (end 156.949258 107.24604) (width 0.25) (layer B.Cu) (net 9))
 (segment (start 157.11678 106.13644) (end 157.11678 104.41432) (width 0.25) (layer B.Cu) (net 9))
 (segment (start 156.849259 106.403961) (end 157.11678 106.13644) (width 0.25) (layer B.Cu) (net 9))
 (segment (start 156.291779 107.224971) (end 156.291779 103.707701) (width 0.25) (layer B.Cu) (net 8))
 (segment (start 156.812848 107.74604) (end 156.291779 107.224971) (width 0.25) (layer B.Cu) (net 8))
 (segment (start 156.291779 103.707701) (end 157.10408 102.8954) (width 0.25) (layer B.Cu) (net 8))
 (segment (start 157.90926 107.74604) (end 156.812848 107.74604) (width 0.25) (layer B.Cu) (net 8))
 (segment (start 155.2321 106.801702) (end 155.2321 104.37622) (width 0.25) (layer B.Cu) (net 7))
 (segment (start 156.676438 108.24604) (end 155.2321 106.801702) (width 0.25) (layer B.Cu) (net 7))
 (segment (start 157.90926 108.24604) (end 156.676438 108.24604) (width 0.25) (layer B.Cu) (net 7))
 (segment (start 154.05862 105.472082) (end 154.05862 102.93604) (width 0.25) (layer B.Cu) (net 6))
 (segment (start 153.249663 106.281039) (end 154.05862 105.472082) (width 0.25) (layer B.Cu) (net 6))
 (segment (start 154.604261 106.281039) (end 153.249663 106.281039) (width 0.25) (layer B.Cu) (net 6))
 (segment (start 154.669261 106.346039) (end 154.604261 106.281039) (width 0.25) (layer B.Cu) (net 6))
 (segment (start 154.669261 106.875273) (end 154.669261 106.346039) (width 0.25) (layer B.Cu) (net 6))
 (segment (start 156.540028 108.74604) (end 154.669261 106.875273) (width 0.25) (layer B.Cu) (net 6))
 (segment (start 157.90926 108.74604) (end 156.540028 108.74604) (width 0.25) (layer B.Cu) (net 6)))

